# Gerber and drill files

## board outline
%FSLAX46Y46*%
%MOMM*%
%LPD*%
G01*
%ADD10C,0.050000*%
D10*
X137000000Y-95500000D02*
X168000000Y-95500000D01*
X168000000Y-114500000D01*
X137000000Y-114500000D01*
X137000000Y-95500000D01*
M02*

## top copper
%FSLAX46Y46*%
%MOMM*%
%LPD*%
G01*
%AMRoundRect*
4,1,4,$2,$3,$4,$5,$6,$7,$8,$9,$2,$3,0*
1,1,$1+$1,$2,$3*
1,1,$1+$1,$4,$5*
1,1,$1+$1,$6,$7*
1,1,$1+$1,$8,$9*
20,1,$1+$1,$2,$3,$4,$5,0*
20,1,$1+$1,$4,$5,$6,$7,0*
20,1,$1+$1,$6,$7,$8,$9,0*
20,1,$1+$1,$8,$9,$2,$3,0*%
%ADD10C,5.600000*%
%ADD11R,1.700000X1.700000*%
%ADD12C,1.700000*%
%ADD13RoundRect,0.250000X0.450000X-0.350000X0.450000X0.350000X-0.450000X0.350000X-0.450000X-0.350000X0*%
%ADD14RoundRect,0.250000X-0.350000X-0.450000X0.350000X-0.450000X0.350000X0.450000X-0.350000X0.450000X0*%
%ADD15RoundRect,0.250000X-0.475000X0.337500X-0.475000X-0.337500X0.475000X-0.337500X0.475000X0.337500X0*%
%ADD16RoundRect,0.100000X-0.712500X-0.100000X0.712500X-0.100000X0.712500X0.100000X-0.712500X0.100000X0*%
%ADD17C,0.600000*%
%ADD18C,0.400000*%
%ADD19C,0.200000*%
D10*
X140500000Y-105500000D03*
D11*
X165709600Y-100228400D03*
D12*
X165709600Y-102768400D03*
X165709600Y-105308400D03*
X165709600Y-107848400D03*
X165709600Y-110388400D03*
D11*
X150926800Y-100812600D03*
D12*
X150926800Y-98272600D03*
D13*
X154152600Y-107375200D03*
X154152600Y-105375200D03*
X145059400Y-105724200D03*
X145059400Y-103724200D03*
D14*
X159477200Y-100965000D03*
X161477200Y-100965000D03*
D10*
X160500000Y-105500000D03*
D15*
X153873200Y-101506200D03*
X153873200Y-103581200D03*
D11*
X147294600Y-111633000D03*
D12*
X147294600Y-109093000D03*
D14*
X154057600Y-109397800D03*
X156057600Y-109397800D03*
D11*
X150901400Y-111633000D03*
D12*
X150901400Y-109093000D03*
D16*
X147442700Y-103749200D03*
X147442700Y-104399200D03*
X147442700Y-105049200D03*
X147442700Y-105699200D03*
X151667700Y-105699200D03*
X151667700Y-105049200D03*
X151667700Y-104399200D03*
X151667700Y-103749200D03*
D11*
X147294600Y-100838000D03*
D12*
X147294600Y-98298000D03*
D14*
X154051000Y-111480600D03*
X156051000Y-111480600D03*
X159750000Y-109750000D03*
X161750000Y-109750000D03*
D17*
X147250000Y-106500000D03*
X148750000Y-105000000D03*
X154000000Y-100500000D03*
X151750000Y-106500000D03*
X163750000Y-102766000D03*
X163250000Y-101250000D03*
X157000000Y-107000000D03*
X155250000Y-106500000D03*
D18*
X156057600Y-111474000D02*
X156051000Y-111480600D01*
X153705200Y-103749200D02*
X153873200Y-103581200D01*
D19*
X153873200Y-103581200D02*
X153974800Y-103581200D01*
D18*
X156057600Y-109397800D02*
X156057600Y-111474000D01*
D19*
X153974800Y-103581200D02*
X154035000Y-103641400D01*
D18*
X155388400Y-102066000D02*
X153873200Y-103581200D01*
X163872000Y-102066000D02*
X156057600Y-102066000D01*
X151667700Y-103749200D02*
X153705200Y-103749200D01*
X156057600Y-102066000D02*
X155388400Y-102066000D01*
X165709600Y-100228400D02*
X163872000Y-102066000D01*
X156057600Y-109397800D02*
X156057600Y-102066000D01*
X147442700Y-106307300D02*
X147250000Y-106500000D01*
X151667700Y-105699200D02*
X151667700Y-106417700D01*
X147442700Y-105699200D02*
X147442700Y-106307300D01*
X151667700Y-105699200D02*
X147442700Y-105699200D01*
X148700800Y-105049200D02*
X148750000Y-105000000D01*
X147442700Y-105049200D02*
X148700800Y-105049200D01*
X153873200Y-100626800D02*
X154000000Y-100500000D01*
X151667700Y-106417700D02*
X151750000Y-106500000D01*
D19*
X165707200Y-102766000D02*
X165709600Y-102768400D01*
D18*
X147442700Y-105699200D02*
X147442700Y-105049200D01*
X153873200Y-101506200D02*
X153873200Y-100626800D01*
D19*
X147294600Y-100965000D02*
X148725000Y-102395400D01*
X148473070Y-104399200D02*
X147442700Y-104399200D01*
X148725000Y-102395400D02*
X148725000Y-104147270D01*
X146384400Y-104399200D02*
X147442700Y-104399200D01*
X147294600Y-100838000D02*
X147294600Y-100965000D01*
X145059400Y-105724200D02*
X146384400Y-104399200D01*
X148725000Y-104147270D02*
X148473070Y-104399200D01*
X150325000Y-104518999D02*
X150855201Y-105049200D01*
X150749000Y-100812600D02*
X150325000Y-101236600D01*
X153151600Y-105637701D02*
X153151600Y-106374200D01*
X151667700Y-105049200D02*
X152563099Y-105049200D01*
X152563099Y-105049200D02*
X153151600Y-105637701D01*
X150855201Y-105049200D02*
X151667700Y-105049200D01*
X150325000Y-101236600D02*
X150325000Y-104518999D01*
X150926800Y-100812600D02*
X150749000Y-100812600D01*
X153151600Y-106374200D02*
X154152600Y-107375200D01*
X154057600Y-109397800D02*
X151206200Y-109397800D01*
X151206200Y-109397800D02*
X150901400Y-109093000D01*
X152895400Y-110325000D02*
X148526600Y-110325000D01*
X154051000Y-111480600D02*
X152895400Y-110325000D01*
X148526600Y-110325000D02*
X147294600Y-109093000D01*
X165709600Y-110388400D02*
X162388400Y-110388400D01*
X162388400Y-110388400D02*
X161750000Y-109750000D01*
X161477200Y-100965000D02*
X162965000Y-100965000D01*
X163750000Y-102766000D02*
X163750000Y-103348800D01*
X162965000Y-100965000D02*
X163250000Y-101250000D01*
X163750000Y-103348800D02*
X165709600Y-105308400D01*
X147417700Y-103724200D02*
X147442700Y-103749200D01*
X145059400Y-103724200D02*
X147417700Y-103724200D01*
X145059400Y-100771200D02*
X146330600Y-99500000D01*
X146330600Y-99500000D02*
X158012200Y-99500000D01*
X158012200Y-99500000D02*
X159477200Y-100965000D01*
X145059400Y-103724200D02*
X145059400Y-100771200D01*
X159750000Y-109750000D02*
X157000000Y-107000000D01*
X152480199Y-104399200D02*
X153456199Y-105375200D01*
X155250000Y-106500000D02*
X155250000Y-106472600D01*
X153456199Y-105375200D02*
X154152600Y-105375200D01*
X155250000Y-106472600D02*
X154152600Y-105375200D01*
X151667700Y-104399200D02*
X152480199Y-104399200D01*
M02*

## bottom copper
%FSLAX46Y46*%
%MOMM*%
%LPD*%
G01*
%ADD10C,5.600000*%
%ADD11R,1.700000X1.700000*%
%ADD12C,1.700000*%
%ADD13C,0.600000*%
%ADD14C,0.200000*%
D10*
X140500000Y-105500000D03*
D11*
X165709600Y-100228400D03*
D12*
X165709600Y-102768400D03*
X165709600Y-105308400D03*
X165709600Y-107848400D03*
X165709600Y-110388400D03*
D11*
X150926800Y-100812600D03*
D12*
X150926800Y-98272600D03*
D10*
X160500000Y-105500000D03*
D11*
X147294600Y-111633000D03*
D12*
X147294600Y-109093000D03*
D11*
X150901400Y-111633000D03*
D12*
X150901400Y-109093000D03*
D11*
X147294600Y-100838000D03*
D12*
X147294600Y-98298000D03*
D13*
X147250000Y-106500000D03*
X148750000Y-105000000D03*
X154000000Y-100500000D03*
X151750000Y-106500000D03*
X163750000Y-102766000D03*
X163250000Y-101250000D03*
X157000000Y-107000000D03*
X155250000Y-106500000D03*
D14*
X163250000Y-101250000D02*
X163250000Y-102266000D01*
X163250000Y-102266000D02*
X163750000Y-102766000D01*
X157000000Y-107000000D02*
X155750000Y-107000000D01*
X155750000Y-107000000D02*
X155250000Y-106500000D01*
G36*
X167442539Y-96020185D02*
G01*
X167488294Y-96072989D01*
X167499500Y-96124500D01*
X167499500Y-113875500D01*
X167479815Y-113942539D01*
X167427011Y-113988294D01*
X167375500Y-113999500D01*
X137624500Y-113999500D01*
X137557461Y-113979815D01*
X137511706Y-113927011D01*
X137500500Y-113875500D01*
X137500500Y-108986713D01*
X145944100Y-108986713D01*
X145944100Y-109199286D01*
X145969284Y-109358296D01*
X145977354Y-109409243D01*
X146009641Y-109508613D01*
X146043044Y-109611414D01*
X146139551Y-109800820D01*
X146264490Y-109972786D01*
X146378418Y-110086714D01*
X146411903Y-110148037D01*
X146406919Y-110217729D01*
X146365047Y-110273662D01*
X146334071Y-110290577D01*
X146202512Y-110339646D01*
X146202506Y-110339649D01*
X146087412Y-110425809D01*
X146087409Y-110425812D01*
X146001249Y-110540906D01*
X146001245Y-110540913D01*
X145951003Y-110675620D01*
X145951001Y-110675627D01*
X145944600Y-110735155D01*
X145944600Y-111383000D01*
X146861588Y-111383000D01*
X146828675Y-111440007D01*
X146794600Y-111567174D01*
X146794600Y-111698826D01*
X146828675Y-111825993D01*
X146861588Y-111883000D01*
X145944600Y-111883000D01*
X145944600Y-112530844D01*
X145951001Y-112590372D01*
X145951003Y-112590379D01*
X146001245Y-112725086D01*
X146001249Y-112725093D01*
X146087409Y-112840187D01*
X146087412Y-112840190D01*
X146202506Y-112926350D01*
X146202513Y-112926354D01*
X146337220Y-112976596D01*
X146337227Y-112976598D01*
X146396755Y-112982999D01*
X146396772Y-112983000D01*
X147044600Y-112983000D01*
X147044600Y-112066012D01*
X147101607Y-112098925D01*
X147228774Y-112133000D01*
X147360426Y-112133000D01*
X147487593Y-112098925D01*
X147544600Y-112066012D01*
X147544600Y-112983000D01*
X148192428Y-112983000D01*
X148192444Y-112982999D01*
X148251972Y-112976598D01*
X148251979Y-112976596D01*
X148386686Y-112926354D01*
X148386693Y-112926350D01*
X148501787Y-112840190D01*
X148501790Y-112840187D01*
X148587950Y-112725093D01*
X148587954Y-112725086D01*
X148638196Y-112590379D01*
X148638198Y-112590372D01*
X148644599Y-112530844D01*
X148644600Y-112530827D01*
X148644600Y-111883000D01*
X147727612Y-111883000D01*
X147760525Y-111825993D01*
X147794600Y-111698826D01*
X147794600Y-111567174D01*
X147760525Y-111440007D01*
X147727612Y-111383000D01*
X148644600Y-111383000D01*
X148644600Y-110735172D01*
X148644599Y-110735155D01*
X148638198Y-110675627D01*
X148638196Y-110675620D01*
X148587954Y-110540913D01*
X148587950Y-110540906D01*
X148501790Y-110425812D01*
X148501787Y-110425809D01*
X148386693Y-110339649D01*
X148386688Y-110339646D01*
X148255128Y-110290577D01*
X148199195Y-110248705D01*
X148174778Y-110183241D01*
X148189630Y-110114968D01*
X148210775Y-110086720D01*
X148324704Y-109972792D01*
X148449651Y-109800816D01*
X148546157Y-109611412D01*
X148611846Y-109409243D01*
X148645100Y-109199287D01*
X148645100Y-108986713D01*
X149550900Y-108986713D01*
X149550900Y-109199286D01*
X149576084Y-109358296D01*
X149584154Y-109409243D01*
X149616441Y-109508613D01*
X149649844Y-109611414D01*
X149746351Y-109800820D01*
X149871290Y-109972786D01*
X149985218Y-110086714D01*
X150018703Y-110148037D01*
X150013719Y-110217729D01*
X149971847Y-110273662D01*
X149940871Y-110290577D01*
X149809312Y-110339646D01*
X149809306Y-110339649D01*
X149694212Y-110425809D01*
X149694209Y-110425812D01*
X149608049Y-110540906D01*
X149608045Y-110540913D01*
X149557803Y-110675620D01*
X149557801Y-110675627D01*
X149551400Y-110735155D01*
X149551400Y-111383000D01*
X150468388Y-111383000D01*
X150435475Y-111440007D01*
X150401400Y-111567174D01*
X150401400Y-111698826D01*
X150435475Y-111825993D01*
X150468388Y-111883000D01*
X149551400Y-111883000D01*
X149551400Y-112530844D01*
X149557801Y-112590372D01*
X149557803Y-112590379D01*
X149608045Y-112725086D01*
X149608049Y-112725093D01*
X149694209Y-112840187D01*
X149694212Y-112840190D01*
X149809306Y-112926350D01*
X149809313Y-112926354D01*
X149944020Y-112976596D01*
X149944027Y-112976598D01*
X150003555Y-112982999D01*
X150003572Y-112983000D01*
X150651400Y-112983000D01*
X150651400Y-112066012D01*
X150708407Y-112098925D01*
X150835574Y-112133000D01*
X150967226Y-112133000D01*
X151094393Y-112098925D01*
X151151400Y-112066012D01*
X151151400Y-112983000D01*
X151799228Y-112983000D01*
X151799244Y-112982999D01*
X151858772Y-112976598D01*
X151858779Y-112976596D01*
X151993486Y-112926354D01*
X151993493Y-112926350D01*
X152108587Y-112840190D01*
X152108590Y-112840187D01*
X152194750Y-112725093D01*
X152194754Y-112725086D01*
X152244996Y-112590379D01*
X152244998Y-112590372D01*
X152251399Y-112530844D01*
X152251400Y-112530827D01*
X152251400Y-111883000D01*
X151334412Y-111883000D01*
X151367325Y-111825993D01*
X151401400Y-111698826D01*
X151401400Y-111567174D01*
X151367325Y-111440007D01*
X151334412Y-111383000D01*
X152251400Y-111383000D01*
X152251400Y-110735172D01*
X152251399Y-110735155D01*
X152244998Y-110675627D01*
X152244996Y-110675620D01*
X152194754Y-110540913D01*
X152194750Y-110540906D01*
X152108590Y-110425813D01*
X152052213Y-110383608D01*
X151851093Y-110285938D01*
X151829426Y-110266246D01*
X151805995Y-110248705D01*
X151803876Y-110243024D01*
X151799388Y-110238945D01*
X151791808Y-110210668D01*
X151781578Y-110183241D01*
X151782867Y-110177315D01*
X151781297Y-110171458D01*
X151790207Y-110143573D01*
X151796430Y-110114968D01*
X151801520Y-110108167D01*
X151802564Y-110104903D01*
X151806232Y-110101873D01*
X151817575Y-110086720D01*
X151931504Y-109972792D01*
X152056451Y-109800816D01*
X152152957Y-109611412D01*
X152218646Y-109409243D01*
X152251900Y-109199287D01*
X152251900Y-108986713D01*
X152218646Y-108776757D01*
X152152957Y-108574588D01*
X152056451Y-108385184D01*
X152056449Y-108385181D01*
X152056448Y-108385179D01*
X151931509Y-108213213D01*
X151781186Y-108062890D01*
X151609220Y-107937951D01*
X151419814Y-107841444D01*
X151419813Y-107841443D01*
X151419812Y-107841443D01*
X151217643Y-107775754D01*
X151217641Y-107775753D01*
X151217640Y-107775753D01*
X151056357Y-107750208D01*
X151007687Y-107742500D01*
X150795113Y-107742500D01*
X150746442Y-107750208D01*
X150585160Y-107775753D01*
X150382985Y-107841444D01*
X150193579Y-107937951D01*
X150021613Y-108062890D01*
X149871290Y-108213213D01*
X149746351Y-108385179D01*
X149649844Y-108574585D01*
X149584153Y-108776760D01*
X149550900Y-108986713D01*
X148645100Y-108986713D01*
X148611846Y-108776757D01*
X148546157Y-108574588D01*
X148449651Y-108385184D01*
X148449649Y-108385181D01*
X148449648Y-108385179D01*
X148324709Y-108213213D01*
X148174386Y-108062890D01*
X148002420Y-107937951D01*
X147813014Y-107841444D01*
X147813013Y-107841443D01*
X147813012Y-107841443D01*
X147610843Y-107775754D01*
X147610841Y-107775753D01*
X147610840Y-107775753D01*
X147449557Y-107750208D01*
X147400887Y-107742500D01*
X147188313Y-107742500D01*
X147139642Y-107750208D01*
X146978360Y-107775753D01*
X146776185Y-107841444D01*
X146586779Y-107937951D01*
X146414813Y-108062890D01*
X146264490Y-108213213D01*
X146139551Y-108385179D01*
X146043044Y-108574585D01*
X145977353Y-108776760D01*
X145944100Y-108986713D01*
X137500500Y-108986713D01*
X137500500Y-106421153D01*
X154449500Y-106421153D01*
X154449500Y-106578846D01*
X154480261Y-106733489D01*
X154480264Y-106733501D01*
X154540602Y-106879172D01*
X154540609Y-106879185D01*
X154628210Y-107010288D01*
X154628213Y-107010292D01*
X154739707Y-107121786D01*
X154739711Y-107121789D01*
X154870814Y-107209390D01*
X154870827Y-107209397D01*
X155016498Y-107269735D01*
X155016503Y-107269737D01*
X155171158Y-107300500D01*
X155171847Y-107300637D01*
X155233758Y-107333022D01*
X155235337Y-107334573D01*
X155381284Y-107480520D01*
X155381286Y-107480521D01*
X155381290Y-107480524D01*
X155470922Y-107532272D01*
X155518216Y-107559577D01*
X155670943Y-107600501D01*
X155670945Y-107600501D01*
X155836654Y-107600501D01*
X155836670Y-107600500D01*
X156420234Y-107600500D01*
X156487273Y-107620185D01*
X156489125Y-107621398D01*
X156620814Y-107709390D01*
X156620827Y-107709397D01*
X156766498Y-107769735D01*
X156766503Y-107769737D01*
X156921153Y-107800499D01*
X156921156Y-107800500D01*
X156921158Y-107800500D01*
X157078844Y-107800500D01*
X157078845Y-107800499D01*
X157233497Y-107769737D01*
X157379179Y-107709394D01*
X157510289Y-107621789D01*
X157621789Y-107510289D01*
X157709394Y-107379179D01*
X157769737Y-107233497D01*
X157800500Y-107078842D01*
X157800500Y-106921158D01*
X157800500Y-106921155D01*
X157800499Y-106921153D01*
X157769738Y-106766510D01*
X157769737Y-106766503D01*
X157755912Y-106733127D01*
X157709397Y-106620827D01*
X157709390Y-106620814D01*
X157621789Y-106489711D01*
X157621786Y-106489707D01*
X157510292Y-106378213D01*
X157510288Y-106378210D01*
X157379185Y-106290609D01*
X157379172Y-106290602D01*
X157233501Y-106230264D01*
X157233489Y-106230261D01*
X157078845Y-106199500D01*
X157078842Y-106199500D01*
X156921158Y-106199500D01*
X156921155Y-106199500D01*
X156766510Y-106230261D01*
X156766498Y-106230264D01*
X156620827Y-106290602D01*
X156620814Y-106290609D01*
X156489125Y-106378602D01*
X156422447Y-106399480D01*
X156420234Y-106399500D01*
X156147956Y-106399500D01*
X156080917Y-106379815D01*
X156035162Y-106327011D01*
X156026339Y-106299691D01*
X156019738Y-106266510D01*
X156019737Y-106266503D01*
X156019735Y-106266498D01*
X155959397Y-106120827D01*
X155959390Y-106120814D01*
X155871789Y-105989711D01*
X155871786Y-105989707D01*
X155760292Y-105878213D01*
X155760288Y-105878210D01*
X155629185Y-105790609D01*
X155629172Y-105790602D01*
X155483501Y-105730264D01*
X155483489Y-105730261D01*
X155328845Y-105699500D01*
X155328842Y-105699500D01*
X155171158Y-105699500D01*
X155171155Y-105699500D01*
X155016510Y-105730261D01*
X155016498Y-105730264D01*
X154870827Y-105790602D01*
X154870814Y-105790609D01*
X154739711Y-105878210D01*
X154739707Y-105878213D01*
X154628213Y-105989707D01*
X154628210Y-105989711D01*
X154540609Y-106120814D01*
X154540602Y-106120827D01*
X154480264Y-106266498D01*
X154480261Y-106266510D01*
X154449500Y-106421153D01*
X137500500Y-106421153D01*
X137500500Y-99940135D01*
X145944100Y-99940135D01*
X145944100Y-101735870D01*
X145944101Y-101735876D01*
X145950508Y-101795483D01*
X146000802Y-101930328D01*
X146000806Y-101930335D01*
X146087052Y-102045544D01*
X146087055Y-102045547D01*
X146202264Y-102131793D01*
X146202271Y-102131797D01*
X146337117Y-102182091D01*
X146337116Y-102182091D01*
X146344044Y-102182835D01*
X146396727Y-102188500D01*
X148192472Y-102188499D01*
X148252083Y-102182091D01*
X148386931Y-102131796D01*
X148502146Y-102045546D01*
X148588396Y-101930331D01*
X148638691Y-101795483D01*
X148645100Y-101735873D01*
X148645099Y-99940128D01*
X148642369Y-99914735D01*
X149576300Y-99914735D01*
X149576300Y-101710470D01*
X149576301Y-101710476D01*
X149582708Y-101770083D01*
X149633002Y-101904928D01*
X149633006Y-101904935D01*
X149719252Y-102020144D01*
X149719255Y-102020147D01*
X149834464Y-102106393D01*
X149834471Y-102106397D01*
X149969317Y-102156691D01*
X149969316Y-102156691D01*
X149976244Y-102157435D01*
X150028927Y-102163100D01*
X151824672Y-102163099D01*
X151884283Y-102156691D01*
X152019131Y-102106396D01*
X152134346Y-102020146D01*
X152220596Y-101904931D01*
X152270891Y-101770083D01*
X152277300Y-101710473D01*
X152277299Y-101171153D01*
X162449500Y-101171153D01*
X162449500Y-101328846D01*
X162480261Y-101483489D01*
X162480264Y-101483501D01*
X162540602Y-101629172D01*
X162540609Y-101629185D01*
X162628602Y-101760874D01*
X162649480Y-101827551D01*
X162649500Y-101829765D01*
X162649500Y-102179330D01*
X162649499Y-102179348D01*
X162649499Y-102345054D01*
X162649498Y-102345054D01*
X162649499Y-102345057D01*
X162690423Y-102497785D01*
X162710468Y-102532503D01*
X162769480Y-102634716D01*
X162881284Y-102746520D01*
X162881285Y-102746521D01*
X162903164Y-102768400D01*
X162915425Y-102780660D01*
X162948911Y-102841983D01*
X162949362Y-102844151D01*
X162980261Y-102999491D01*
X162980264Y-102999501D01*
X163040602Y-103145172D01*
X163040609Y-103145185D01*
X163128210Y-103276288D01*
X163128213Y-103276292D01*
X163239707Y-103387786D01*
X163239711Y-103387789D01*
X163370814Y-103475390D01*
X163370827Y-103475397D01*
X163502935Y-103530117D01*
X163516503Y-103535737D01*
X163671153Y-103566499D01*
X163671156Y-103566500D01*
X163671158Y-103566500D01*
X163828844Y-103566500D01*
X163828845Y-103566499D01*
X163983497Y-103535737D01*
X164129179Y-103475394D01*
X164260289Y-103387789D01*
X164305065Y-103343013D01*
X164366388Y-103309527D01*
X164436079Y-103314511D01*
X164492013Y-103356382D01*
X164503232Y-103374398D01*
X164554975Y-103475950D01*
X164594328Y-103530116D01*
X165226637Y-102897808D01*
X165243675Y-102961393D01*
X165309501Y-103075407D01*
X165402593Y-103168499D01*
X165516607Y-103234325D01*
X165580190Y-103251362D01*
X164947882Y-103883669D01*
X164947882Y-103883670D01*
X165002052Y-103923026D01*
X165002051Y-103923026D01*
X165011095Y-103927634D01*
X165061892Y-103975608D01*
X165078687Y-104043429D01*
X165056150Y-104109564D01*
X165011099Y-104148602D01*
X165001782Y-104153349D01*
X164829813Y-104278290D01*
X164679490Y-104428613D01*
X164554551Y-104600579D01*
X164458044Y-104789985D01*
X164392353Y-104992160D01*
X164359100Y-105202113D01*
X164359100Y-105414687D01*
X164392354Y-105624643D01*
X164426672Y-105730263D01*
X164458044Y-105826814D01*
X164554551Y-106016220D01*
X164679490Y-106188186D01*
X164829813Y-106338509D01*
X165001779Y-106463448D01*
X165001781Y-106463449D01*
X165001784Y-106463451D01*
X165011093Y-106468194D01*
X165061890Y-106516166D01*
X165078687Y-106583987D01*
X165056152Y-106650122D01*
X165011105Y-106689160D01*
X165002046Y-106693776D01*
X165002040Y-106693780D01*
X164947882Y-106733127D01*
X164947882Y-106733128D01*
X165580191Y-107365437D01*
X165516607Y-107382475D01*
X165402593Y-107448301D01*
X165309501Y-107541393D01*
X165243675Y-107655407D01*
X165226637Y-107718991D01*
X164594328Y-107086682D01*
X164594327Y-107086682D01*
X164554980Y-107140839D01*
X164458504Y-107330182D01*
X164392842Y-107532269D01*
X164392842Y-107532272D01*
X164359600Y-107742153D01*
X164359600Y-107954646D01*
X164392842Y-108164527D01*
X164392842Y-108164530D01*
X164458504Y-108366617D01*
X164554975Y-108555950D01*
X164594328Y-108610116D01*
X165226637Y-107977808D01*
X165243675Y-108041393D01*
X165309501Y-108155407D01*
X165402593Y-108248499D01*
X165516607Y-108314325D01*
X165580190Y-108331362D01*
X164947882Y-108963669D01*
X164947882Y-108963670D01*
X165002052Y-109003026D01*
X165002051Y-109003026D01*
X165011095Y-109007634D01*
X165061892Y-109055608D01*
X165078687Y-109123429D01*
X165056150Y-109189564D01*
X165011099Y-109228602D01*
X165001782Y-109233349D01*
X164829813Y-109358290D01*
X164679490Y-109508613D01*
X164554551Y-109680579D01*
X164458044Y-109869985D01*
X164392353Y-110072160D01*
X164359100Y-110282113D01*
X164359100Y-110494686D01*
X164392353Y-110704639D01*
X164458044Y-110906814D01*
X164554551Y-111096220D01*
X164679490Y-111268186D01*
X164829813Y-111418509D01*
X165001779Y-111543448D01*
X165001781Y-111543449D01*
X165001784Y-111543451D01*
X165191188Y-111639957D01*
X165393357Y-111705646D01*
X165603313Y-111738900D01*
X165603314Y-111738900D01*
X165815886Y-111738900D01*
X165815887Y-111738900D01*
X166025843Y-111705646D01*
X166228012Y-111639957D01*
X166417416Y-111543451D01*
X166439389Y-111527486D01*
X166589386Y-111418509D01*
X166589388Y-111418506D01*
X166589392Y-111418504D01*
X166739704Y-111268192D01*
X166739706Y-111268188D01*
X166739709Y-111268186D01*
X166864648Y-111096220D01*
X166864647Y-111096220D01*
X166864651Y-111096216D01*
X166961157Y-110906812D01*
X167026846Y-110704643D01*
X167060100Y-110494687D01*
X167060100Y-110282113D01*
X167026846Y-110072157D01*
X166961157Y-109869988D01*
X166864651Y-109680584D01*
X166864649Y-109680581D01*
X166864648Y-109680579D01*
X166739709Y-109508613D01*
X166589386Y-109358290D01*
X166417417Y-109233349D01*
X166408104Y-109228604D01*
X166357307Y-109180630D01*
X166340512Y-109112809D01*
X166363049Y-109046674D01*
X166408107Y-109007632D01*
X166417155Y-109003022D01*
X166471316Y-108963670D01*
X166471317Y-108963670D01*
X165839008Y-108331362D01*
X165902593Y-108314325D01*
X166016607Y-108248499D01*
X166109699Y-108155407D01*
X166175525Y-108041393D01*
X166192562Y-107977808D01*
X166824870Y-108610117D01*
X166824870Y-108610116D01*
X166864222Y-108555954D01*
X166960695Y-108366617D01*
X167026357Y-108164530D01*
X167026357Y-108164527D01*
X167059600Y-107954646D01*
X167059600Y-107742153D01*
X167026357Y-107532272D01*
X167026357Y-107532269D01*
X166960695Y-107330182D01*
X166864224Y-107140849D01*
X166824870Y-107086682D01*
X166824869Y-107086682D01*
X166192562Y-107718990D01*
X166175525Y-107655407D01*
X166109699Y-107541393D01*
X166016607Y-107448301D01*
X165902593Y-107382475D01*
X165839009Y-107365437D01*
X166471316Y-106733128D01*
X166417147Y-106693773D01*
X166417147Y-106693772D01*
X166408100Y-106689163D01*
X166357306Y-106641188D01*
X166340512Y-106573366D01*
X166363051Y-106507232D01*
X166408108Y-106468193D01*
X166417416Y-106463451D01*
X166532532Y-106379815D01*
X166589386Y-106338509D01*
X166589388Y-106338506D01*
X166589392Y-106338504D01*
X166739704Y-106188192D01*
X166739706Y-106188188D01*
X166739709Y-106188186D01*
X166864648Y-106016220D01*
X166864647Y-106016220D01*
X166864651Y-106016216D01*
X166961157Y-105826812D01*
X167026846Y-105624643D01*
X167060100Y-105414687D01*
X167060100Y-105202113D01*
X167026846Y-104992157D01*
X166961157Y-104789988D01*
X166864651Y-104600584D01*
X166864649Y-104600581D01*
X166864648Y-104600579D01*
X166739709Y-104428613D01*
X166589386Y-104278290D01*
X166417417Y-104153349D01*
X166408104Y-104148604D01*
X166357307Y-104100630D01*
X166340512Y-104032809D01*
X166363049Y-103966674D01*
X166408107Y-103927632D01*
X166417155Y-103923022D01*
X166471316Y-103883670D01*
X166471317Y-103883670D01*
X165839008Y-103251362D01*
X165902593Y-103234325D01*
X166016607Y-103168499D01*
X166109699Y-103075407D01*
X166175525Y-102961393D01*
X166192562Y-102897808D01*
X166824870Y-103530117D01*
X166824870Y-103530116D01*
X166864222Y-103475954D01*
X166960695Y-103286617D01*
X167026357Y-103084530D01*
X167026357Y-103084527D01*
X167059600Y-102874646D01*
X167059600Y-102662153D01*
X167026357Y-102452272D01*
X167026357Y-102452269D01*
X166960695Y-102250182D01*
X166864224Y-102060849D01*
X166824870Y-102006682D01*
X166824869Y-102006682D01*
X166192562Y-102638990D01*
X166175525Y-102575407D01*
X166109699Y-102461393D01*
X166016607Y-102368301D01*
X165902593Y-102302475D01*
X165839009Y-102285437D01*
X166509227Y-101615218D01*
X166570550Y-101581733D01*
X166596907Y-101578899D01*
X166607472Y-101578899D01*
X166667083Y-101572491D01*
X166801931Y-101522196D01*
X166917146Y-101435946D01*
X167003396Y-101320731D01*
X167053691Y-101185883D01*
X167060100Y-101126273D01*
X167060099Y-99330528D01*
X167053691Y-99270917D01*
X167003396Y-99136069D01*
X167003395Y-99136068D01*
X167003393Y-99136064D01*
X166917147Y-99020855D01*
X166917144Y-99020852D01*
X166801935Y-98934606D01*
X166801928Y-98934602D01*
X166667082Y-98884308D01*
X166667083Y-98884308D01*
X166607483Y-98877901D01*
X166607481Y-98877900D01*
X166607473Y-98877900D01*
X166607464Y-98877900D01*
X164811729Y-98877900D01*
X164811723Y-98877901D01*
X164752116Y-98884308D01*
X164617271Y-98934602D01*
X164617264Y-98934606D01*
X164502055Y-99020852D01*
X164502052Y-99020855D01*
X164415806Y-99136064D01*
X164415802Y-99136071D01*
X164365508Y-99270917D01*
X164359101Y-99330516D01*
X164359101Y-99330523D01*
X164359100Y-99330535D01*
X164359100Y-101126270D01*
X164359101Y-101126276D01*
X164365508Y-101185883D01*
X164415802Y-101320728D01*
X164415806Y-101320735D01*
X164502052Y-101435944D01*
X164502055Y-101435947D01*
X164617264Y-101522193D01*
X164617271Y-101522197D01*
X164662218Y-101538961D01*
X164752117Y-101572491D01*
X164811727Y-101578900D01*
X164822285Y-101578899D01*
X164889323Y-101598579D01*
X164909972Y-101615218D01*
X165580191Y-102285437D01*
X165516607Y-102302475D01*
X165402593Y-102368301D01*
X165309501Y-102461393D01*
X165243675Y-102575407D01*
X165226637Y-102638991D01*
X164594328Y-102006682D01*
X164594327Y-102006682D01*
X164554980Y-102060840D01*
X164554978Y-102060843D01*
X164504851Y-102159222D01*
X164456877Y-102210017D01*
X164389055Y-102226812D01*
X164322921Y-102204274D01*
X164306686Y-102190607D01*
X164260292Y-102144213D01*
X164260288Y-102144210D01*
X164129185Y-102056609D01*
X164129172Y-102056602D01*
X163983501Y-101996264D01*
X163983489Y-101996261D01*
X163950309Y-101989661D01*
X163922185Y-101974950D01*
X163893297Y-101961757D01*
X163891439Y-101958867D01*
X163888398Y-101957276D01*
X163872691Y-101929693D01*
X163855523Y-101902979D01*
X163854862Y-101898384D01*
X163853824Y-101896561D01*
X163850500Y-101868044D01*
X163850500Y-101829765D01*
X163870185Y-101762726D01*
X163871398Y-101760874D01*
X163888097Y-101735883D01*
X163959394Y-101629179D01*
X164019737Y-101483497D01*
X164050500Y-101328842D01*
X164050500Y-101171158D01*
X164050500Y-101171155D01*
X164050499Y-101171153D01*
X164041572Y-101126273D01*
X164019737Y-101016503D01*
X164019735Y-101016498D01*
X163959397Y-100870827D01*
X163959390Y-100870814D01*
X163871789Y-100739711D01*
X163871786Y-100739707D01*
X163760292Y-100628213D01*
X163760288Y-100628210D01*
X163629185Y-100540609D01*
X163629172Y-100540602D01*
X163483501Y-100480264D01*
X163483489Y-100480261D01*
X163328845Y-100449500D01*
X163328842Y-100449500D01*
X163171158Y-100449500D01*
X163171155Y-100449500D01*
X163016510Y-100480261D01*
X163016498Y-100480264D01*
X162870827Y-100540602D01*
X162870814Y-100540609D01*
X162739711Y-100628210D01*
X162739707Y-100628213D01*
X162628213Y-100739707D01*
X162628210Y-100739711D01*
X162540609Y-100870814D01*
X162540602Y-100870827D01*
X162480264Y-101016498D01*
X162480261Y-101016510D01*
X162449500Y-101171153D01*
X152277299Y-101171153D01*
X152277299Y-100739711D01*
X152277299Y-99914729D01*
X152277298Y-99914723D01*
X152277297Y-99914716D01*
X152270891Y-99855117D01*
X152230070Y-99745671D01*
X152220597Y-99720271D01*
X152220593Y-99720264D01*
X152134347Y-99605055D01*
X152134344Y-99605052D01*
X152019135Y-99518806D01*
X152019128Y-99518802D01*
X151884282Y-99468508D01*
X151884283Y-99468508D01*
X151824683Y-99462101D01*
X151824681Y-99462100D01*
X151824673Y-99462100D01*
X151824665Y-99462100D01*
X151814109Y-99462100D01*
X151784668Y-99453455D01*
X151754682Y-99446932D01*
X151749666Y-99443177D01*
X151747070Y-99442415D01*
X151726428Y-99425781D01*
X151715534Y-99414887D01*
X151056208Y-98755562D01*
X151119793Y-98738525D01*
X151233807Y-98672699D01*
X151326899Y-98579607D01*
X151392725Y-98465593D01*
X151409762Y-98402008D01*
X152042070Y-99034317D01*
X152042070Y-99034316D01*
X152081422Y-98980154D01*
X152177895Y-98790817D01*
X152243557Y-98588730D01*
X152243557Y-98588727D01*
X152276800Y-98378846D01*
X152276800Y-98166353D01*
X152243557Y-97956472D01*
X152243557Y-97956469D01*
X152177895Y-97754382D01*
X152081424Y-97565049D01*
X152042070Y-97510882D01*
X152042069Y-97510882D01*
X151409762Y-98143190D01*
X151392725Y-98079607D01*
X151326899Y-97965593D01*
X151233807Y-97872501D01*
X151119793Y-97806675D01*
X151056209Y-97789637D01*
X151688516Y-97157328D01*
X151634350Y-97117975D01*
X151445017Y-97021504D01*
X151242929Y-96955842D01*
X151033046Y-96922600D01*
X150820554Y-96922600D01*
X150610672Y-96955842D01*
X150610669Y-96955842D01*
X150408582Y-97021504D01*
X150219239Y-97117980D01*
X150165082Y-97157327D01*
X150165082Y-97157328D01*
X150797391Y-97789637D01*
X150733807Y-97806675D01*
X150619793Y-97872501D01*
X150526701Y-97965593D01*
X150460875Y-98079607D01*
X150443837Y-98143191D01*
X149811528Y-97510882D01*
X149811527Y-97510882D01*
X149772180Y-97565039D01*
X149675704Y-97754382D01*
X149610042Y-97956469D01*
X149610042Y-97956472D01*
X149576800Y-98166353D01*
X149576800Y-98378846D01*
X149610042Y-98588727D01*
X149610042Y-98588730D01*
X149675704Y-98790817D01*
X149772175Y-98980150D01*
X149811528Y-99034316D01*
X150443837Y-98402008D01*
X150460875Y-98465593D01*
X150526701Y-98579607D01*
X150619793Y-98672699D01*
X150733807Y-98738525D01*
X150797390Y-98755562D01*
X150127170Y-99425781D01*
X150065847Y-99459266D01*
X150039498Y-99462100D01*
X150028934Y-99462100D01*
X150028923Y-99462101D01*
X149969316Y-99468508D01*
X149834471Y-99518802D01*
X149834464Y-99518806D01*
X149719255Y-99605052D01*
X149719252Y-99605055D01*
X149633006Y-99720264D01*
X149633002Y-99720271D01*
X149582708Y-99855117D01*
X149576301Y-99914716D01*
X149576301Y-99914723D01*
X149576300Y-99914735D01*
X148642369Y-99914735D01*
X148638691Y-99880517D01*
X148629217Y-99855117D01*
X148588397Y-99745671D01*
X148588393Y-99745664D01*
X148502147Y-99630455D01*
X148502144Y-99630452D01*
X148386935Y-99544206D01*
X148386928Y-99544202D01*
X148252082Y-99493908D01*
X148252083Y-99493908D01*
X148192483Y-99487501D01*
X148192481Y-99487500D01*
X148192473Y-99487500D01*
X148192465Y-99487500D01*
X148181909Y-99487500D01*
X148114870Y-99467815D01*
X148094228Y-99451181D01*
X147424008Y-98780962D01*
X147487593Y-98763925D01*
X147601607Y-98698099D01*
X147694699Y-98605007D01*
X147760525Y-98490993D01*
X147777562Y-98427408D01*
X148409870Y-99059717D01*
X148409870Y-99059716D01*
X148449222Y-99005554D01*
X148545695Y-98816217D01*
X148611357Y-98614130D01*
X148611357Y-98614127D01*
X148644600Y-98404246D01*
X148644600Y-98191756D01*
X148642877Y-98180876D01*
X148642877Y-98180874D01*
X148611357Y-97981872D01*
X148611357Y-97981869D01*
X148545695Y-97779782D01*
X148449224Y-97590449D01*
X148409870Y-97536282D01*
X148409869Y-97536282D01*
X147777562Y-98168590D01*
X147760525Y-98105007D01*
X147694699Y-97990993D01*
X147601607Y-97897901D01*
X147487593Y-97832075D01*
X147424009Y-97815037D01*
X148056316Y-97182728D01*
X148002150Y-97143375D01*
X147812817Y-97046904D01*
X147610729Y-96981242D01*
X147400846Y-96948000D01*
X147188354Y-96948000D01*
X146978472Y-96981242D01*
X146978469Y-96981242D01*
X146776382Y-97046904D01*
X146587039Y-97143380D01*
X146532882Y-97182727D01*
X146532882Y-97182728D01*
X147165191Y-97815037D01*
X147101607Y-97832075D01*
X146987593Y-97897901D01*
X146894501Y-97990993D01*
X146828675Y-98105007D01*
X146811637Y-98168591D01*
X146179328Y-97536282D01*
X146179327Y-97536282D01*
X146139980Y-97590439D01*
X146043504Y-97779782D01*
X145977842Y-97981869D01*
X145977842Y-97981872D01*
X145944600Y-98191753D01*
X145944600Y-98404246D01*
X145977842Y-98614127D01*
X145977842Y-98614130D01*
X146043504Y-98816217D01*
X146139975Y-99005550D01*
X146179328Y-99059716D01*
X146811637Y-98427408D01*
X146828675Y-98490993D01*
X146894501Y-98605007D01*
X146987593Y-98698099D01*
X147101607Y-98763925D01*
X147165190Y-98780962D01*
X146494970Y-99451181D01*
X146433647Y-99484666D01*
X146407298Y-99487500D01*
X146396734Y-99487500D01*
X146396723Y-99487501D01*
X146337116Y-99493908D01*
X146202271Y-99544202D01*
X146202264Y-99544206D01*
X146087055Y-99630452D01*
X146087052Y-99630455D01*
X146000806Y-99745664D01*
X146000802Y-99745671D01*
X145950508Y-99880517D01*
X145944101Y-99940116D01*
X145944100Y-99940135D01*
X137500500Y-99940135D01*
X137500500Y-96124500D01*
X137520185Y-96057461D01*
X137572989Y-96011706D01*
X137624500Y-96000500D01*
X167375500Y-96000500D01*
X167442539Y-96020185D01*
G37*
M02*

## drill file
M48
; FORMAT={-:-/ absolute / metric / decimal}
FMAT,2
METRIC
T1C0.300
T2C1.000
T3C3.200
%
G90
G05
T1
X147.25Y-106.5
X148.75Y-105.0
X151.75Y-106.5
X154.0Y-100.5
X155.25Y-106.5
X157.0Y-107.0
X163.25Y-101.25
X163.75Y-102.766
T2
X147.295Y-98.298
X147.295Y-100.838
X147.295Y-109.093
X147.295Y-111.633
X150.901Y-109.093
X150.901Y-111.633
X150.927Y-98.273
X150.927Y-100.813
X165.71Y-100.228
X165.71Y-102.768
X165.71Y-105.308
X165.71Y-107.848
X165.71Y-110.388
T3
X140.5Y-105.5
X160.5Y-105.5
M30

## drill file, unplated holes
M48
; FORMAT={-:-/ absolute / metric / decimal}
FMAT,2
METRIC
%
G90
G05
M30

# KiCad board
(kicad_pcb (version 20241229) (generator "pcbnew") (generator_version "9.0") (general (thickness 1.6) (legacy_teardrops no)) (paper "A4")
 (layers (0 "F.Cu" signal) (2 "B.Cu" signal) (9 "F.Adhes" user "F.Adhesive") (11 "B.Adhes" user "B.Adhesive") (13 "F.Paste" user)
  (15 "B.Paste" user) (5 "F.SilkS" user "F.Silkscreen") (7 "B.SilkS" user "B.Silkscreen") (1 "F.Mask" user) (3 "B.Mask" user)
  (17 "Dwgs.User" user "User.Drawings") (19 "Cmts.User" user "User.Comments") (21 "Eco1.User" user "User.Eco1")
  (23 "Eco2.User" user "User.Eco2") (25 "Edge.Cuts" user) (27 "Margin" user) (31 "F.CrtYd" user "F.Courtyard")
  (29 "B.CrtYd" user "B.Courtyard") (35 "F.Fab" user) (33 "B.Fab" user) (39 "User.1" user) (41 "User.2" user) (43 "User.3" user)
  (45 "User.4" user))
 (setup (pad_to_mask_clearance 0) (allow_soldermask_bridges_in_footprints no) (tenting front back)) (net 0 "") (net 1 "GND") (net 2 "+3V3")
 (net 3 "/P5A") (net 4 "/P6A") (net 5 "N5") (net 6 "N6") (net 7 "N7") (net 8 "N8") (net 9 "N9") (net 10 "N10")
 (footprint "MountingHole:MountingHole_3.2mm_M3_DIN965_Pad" (layer "F.Cu") (at 140.5 105.5)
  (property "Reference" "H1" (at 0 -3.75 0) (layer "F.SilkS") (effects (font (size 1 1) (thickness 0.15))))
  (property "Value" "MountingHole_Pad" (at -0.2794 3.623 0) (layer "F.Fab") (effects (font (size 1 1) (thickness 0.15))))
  (pad "1" thru_hole circle (at 0 0) (size 5.6 5.6) (drill 3.2) (layers "*.Cu" "*.Mask") (remove_unused_layers no) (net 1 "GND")
   (zone_connect 2)))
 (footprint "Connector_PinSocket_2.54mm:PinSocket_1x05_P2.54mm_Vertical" (layer "F.Cu") (at 165.7096 100.2284)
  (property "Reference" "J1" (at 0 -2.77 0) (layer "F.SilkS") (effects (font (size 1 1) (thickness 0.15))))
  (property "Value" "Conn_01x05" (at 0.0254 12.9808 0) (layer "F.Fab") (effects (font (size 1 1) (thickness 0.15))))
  (pad "1" thru_hole rect (at 0 0) (size 1.7 1.7) (drill 1) (layers "*.Cu" "*.Mask") (remove_unused_layers no) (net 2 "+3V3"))
  (pad "2" thru_hole circle (at 0 2.54) (size 1.7 1.7) (drill 1) (layers "*.Cu" "*.Mask") (remove_unused_layers no) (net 1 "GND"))
  (pad "3" thru_hole circle (at 0 5.08) (size 1.7 1.7) (drill 1) (layers "*.Cu" "*.Mask") (remove_unused_layers no) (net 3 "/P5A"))
  (pad "4" thru_hole circle (at 0 7.62) (size 1.7 1.7) (drill 1) (layers "*.Cu" "*.Mask") (remove_unused_layers no) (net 1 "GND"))
  (pad "5" thru_hole circle (at 0 10.16) (size 1.7 1.7) (drill 1) (layers "*.Cu" "*.Mask") (remove_unused_layers no) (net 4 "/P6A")))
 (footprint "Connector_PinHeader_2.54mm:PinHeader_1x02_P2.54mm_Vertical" (layer "F.Cu") (at 150.9268 100.8126 180)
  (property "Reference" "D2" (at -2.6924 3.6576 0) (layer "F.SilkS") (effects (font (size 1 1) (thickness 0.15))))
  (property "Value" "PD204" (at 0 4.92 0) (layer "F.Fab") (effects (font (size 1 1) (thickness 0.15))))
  (pad "1" thru_hole rect (at 0 0 180) (size 1.7 1.7) (drill 1) (layers "*.Cu" "*.Mask") (remove_unused_layers no) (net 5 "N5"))
  (pad "2" thru_hole circle (at 0 2.54 180) (size 1.7 1.7) (drill 1) (layers "*.Cu" "*.Mask") (remove_unused_layers no) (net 1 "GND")))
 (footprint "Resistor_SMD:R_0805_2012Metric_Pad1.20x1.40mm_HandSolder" (layer "F.Cu") (at 154.1526 106.3752 90)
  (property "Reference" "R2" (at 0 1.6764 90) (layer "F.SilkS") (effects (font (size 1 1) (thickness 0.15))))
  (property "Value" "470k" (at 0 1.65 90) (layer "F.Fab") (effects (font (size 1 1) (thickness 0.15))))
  (pad "1" smd roundrect (at -1 0 90) (size 1.2 1.4) (layers "F.Cu" "F.Mask" "F.Paste") (roundrect_rratio 0.208333) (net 5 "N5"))
  (pad "2" smd roundrect (at 1 0 90) (size 1.2 1.4) (layers "F.Cu" "F.Mask" "F.Paste") (roundrect_rratio 0.208333) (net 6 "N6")))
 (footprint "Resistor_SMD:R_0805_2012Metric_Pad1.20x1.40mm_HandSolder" (layer "F.Cu") (at 145.0594 104.7242 90)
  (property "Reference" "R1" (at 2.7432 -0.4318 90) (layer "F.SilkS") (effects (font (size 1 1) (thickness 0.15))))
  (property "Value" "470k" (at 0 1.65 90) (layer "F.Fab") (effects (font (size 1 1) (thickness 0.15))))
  (pad "1" smd roundrect (at -1 0 90) (size 1.2 1.4) (layers "F.Cu" "F.Mask" "F.Paste") (roundrect_rratio 0.208333) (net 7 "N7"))
  (pad "2" smd roundrect (at 1 0 90) (size 1.2 1.4) (layers "F.Cu" "F.Mask" "F.Paste") (roundrect_rratio 0.208333) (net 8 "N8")))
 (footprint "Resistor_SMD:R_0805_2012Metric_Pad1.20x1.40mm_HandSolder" (layer "F.Cu") (at 160.4772 100.965)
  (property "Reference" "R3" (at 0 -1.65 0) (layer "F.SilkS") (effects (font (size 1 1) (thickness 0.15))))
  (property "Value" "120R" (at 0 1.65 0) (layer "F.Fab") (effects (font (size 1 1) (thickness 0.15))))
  (pad "1" smd roundrect (at -1 0) (size 1.2 1.4) (layers "F.Cu" "F.Mask" "F.Paste") (roundrect_rratio 0.208333) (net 8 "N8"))
  (pad "2" smd roundrect (at 1 0) (size 1.2 1.4) (layers "F.Cu" "F.Mask" "F.Paste") (roundrect_rratio 0.208333) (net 3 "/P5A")))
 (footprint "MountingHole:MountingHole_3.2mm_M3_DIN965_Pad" (layer "F.Cu") (at 160.5 105.5)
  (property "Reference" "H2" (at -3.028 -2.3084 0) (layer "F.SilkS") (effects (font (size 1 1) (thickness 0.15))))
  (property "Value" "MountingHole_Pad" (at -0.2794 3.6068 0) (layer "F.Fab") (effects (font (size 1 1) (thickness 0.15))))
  (pad "1" thru_hole circle (at 0 0) (size 5.6 5.6) (drill 3.2) (layers "*.Cu" "*.Mask") (remove_unused_layers no) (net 1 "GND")
   (zone_connect 2)))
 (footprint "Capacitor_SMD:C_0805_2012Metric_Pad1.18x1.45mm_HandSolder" (layer "F.Cu") (at 153.8732 102.5437 -90)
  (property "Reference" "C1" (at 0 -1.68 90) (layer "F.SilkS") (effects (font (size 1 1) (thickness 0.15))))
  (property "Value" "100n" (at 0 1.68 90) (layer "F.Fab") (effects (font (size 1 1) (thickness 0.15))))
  (pad "1" smd roundrect (at -1.0375 0 270) (size 1.175 1.45) (layers "F.Cu" "F.Mask" "F.Paste") (roundrect_rratio 0.212766) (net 1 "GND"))
  (pad "2" smd roundrect (at 1.0375 0 270) (size 1.175 1.45) (layers "F.Cu" "F.Mask" "F.Paste") (roundrect_rratio 0.212766) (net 2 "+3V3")))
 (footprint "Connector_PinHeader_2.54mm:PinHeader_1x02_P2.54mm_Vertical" (layer "F.Cu") (at 147.2946 111.633 180)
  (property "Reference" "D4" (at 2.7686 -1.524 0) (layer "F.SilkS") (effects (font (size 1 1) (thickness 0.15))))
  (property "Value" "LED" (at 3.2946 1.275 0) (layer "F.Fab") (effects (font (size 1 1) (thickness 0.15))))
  (pad "1" thru_hole rect (at 0 0 180) (size 1.7 1.7) (drill 1) (layers "*.Cu" "*.Mask") (remove_unused_layers no) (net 1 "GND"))
  (pad "2" thru_hole circle (at 0 2.54 180) (size 1.7 1.7) (drill 1) (layers "*.Cu" "*.Mask") (remove_unused_layers no) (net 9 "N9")))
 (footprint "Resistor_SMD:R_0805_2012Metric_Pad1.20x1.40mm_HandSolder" (layer "F.Cu") (at 155.0576 109.3978)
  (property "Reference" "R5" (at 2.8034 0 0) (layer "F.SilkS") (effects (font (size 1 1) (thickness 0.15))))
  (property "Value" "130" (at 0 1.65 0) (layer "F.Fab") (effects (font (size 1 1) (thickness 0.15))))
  (pad "1" smd roundrect (at -1 0) (size 1.2 1.4) (layers "F.Cu" "F.Mask" "F.Paste") (roundrect_rratio 0.208333) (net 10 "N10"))
  (pad "2" smd roundrect (at 1 0) (size 1.2 1.4) (layers "F.Cu" "F.Mask" "F.Paste") (roundrect_rratio 0.208333) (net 2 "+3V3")))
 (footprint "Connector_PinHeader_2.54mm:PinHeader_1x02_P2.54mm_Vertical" (layer "F.Cu") (at 150.9014 111.633 180)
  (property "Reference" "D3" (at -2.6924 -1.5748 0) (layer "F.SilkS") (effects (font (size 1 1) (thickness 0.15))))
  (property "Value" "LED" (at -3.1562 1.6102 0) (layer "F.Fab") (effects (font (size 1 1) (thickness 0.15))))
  (pad "1" thru_hole rect (at 0 0 180) (size 1.7 1.7) (drill 1) (layers "*.Cu" "*.Mask") (remove_unused_layers no) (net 1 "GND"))
  (pad "2" thru_hole circle (at 0 2.54 180) (size 1.7 1.7) (drill 1) (layers "*.Cu" "*.Mask") (remove_unused_layers no) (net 10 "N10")))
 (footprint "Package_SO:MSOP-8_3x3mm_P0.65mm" (layer "F.Cu") (at 149.5552 104.7242)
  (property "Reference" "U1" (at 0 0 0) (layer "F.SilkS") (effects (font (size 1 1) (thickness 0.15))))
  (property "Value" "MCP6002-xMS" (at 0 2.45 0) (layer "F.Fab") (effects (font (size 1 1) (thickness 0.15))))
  (pad "1" smd roundrect (at -2.1125 -0.975) (size 1.625 0.4) (layers "F.Cu" "F.Mask" "F.Paste") (roundrect_rratio 0.25) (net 8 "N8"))
  (pad "2" smd roundrect (at -2.1125 -0.325) (size 1.625 0.4) (layers "F.Cu" "F.Mask" "F.Paste") (roundrect_rratio 0.25) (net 7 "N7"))
  (pad "3" smd roundrect (at -2.1125 0.325) (size 1.625 0.4) (layers "F.Cu" "F.Mask" "F.Paste") (roundrect_rratio 0.25) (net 1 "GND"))
  (pad "4" smd roundrect (at -2.1125 0.975) (size 1.625 0.4) (layers "F.Cu" "F.Mask" "F.Paste") (roundrect_rratio 0.25) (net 1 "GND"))
  (pad "5" smd roundrect (at 2.1125 0.975) (size 1.625 0.4) (layers "F.Cu" "F.Mask" "F.Paste") (roundrect_rratio 0.25) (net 1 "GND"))
  (pad "6" smd roundrect (at 2.1125 0.325) (size 1.625 0.4) (layers "F.Cu" "F.Mask" "F.Paste") (roundrect_rratio 0.25) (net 5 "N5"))
  (pad "7" smd roundrect (at 2.1125 -0.325) (size 1.625 0.4) (layers "F.Cu" "F.Mask" "F.Paste") (roundrect_rratio 0.25) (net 6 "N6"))
  (pad "8" smd roundrect (at 2.1125 -0.975) (size 1.625 0.4) (layers "F.Cu" "F.Mask" "F.Paste") (roundrect_rratio 0.25) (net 2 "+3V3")))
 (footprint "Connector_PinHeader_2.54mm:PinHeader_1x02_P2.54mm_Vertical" (layer "F.Cu") (at 147.2946 100.838 180)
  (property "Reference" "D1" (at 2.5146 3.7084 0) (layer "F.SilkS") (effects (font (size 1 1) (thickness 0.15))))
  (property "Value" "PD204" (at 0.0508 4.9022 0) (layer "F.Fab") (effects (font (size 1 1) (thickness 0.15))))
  (pad "1" thru_hole rect (at 0 0 180) (size 1.7 1.7) (drill 1) (layers "*.Cu" "*.Mask") (remove_unused_layers no) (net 7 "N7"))
  (pad "2" thru_hole circle (at 0 2.54 180) (size 1.7 1.7) (drill 1) (layers "*.Cu" "*.Mask") (remove_unused_layers no) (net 1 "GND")))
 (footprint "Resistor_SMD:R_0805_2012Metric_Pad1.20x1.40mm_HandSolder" (layer "F.Cu") (at 155.051 111.4806)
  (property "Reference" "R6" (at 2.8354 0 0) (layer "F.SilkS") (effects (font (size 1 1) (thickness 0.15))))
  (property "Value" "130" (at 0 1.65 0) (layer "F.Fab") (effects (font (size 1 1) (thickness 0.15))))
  (pad "1" smd roundrect (at -1 0) (size 1.2 1.4) (layers "F.Cu" "F.Mask" "F.Paste") (roundrect_rratio 0.208333) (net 9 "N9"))
  (pad "2" smd roundrect (at 1 0) (size 1.2 1.4) (layers "F.Cu" "F.Mask" "F.Paste") (roundrect_rratio 0.208333) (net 2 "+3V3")))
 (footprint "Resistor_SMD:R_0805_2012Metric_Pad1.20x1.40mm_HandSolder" (layer "F.Cu") (at 160.75 109.75)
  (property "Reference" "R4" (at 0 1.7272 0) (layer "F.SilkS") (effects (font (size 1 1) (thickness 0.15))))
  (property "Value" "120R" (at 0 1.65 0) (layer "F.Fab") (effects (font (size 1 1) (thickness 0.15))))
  (pad "1" smd roundrect (at -1 0) (size 1.2 1.4) (layers "F.Cu" "F.Mask" "F.Paste") (roundrect_rratio 0.208333) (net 6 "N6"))
  (pad "2" smd roundrect (at 1 0) (size 1.2 1.4) (layers "F.Cu" "F.Mask" "F.Paste") (roundrect_rratio 0.208333) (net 4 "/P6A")))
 (gr_rect (start 137 95.5) (end 168 114.5) (stroke (width 0.05) (type default)) (fill no) (layer "Edge.Cuts"))
 (segment (start 156.0576 111.474) (end 156.051 111.4806) (width 0.4) (layer "F.Cu") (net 2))
 (segment (start 155.9464 103.5812) (end 156.0576 103.6924) (width 0.4) (layer "F.Cu") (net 2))
 (segment (start 153.7052 103.7492) (end 153.8732 103.5812) (width 0.4) (layer "F.Cu") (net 2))
 (segment (start 153.8732 103.5812) (end 155.9464 103.5812) (width 0.4) (layer "F.Cu") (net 2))
 (segment (start 153.8732 103.5812) (end 153.9748 103.5812) (width 0.2) (layer "F.Cu") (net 2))
 (segment (start 156.0576 109.3978) (end 156.0576 111.474) (width 0.4) (layer "F.Cu") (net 2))
 (segment (start 153.9748 103.5812) (end 154.035 103.6414) (width 0.2) (layer "F.Cu") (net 2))
 (segment (start 156.0576 109.3978) (end 156.0576 103.6924) (width 0.4) (layer "F.Cu") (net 2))
 (segment (start 151.6677 103.7492) (end 153.7052 103.7492) (width 0.4) (layer "F.Cu") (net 2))
 (segment (start 163.872 102.066) (end 165.7096 100.2284) (width 0.4) (layer "F.Cu") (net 2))
 (segment (start 156.0576 103.6924) (end 157.684 102.066) (width 0.4) (layer "F.Cu") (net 2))
 (segment (start 157.684 102.066) (end 163.872 102.066) (width 0.4) (layer "F.Cu") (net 2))
 (segment (start 147.4427 106.3073) (end 147.25 106.5) (width 0.4) (layer "F.Cu") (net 1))
 (segment (start 151.6677 105.6992) (end 151.6677 106.4177) (width 0.4) (layer "F.Cu") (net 1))
 (segment (start 147.4427 105.6992) (end 147.4427 106.3073) (width 0.4) (layer "F.Cu") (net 1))
 (segment (start 151.6677 105.6992) (end 147.4427 105.6992) (width 0.4) (layer "F.Cu") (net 1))
 (segment (start 148.7008 105.0492) (end 148.75 105) (width 0.4) (layer "F.Cu") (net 1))
 (segment (start 147.4427 105.0492) (end 148.7008 105.0492) (width 0.4) (layer "F.Cu") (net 1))
 (segment (start 153.8732 100.6268) (end 154 100.5) (width 0.4) (layer "F.Cu") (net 1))
 (segment (start 151.6677 106.4177) (end 151.75 106.5) (width 0.4) (layer "F.Cu") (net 1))
 (segment (start 165.7072 102.766) (end 165.7096 102.7684) (width 0.2) (layer "F.Cu") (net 1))
 (segment (start 147.4427 105.6992) (end 147.4427 105.0492) (width 0.4) (layer "F.Cu") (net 1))
 (segment (start 153.8732 101.5062) (end 153.8732 100.6268) (width 0.4) (layer "F.Cu") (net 1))
 (via (at 147.25 106.5) (size 0.6) (drill 0.3) (layers "F.Cu" "B.Cu") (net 1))
 (via (at 148.75 105) (size 0.6) (drill 0.3) (layers "F.Cu" "B.Cu") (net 1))
 (via (at 154 100.5) (size 0.6) (drill 0.3) (layers "F.Cu" "B.Cu") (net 1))
 (via (at 151.75 106.5) (size 0.6) (drill 0.3) (layers "F.Cu" "B.Cu") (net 1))
 (segment (start 147.2946 100.965) (end 148.725 102.3954) (width 0.2) (layer "F.Cu") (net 7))
 (segment (start 148.47307 104.3992) (end 147.4427 104.3992) (width 0.2) (layer "F.Cu") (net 7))
 (segment (start 148.725 102.3954) (end 148.725 104.14727) (width 0.2) (layer "F.Cu") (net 7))
 (segment (start 146.3844 104.3992) (end 147.4427 104.3992) (width 0.2) (layer "F.Cu") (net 7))
 (segment (start 147.2946 100.838) (end 147.2946 100.965) (width 0.2) (layer "F.Cu") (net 7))
 (segment (start 145.0594 105.7242) (end 146.3844 104.3992) (width 0.2) (layer "F.Cu") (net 7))
 (segment (start 148.725 104.14727) (end 148.47307 104.3992) (width 0.2) (layer "F.Cu") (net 7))
 (segment (start 150.325 104.518999) (end 150.855201 105.0492) (width 0.2) (layer "F.Cu") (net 5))
 (segment (start 150.749 100.8126) (end 150.325 101.2366) (width 0.2) (layer "F.Cu") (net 5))
 (segment (start 153.1516 105.637701) (end 153.1516 106.3742) (width 0.2) (layer "F.Cu") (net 5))
 (segment (start 151.6677 105.0492) (end 152.563099 105.0492) (width 0.2) (layer "F.Cu") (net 5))
 (segment (start 152.563099 105.0492) (end 153.1516 105.637701) (width 0.2) (layer "F.Cu") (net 5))
 (segment (start 150.855201 105.0492) (end 151.6677 105.0492) (width 0.2) (layer "F.Cu") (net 5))
 (segment (start 150.325 101.2366) (end 150.325 104.518999) (width 0.2) (layer "F.Cu") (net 5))
 (segment (start 150.9268 100.8126) (end 150.749 100.8126) (width 0.2) (layer "F.Cu") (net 5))
 (segment (start 153.1516 106.3742) (end 154.1526 107.3752) (width 0.2) (layer "F.Cu") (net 5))
 (segment (start 154.0576 109.3978) (end 151.2062 109.3978) (width 0.2) (layer "F.Cu") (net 10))
 (segment (start 151.2062 109.3978) (end 150.9014 109.093) (width 0.2) (layer "F.Cu") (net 10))
 (segment (start 152.8954 110.325) (end 148.5266 110.325) (width 0.2) (layer "F.Cu") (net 9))
 (segment (start 154.051 111.4806) (end 152.8954 110.325) (width 0.2) (layer "F.Cu") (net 9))
 (segment (start 148.5266 110.325) (end 147.2946 109.093) (width 0.2) (layer "F.Cu") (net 9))
 (segment (start 165.7096 110.3884) (end 162.3884 110.3884) (width 0.2) (layer "F.Cu") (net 4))
 (segment (start 162.3884 110.3884) (end 161.75 109.75) (width 0.2) (layer "F.Cu") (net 4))
 (segment (start 161.4772 100.965) (end 162.965 100.965) (width 0.2) (layer "F.Cu") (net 3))
 (segment (start 163.75 102.766) (end 163.75 103.3488) (width 0.2) (layer "F.Cu") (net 3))
 (segment (start 162.965 100.965) (end 163.25 101.25) (width 0.2) (layer "F.Cu") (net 3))
 (segment (start 163.75 103.3488) (end 165.7096 105.3084) (width 0.2) (layer "F.Cu") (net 3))
 (via (at 163.75 102.766) (size 0.6) (drill 0.3) (layers "F.Cu" "B.Cu") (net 3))
 (via (at 163.25 101.25) (size 0.6) (drill 0.3) (layers "F.Cu" "B.Cu") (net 3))
 (segment (start 163.25 101.25) (end 163.25 102.266) (width 0.2) (layer "B.Cu") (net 3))
 (segment (start 163.25 102.266) (end 163.75 102.766) (width 0.2) (layer "B.Cu") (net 3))
 (segment (start 147.4177 103.7242) (end 147.4427 103.7492) (width 0.2) (layer "F.Cu") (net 8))
 (segment (start 145.0594 103.7242) (end 147.4177 103.7242) (width 0.2) (layer "F.Cu") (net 8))
 (segment (start 145.0594 100.7712) (end 146.3306 99.5) (width 0.2) (layer "F.Cu") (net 8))
 (segment (start 146.3306 99.5) (end 158.0122 99.5) (width 0.2) (layer "F.Cu") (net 8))
 (segment (start 158.0122 99.5) (end 159.4772 100.965) (width 0.2) (layer "F.Cu") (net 8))
 (segment (start 145.0594 103.7242) (end 145.0594 100.7712) (width 0.2) (layer "F.Cu") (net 8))
 (segment (start 159.75 109.75) (end 157 107) (width 0.2) (layer "F.Cu") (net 6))
 (segment (start 152.480199 104.3992) (end 153.456199 105.3752) (width 0.2) (layer "F.Cu") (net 6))
 (segment (start 155.25 106.5) (end 155.25 106.4726) (width 0.2) (layer "F.Cu") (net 6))
 (segment (start 153.456199 105.3752) (end 154.1526 105.3752) (width 0.2) (layer "F.Cu") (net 6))
 (segment (start 155.25 106.4726) (end 154.1526 105.3752) (width 0.2) (layer "F.Cu") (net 6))
 (segment (start 151.6677 104.3992) (end 152.480199 104.3992) (width 0.2) (layer "F.Cu") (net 6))
 (via (at 157 107) (size 0.6) (drill 0.3) (layers "F.Cu" "B.Cu") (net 6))
 (via (at 155.25 106.5) (size 0.6) (drill 0.3) (layers "F.Cu" "B.Cu") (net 6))
 (segment (start 157 107) (end 155.75 107) (width 0.2) (layer "B.Cu") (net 6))
 (segment (start 155.75 107) (end 155.25 106.5) (width 0.2) (layer "B.Cu") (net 6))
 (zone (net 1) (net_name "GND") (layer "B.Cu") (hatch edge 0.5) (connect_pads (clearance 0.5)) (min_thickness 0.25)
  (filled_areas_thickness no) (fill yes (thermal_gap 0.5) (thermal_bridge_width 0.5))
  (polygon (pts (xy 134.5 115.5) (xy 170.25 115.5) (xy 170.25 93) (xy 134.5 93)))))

